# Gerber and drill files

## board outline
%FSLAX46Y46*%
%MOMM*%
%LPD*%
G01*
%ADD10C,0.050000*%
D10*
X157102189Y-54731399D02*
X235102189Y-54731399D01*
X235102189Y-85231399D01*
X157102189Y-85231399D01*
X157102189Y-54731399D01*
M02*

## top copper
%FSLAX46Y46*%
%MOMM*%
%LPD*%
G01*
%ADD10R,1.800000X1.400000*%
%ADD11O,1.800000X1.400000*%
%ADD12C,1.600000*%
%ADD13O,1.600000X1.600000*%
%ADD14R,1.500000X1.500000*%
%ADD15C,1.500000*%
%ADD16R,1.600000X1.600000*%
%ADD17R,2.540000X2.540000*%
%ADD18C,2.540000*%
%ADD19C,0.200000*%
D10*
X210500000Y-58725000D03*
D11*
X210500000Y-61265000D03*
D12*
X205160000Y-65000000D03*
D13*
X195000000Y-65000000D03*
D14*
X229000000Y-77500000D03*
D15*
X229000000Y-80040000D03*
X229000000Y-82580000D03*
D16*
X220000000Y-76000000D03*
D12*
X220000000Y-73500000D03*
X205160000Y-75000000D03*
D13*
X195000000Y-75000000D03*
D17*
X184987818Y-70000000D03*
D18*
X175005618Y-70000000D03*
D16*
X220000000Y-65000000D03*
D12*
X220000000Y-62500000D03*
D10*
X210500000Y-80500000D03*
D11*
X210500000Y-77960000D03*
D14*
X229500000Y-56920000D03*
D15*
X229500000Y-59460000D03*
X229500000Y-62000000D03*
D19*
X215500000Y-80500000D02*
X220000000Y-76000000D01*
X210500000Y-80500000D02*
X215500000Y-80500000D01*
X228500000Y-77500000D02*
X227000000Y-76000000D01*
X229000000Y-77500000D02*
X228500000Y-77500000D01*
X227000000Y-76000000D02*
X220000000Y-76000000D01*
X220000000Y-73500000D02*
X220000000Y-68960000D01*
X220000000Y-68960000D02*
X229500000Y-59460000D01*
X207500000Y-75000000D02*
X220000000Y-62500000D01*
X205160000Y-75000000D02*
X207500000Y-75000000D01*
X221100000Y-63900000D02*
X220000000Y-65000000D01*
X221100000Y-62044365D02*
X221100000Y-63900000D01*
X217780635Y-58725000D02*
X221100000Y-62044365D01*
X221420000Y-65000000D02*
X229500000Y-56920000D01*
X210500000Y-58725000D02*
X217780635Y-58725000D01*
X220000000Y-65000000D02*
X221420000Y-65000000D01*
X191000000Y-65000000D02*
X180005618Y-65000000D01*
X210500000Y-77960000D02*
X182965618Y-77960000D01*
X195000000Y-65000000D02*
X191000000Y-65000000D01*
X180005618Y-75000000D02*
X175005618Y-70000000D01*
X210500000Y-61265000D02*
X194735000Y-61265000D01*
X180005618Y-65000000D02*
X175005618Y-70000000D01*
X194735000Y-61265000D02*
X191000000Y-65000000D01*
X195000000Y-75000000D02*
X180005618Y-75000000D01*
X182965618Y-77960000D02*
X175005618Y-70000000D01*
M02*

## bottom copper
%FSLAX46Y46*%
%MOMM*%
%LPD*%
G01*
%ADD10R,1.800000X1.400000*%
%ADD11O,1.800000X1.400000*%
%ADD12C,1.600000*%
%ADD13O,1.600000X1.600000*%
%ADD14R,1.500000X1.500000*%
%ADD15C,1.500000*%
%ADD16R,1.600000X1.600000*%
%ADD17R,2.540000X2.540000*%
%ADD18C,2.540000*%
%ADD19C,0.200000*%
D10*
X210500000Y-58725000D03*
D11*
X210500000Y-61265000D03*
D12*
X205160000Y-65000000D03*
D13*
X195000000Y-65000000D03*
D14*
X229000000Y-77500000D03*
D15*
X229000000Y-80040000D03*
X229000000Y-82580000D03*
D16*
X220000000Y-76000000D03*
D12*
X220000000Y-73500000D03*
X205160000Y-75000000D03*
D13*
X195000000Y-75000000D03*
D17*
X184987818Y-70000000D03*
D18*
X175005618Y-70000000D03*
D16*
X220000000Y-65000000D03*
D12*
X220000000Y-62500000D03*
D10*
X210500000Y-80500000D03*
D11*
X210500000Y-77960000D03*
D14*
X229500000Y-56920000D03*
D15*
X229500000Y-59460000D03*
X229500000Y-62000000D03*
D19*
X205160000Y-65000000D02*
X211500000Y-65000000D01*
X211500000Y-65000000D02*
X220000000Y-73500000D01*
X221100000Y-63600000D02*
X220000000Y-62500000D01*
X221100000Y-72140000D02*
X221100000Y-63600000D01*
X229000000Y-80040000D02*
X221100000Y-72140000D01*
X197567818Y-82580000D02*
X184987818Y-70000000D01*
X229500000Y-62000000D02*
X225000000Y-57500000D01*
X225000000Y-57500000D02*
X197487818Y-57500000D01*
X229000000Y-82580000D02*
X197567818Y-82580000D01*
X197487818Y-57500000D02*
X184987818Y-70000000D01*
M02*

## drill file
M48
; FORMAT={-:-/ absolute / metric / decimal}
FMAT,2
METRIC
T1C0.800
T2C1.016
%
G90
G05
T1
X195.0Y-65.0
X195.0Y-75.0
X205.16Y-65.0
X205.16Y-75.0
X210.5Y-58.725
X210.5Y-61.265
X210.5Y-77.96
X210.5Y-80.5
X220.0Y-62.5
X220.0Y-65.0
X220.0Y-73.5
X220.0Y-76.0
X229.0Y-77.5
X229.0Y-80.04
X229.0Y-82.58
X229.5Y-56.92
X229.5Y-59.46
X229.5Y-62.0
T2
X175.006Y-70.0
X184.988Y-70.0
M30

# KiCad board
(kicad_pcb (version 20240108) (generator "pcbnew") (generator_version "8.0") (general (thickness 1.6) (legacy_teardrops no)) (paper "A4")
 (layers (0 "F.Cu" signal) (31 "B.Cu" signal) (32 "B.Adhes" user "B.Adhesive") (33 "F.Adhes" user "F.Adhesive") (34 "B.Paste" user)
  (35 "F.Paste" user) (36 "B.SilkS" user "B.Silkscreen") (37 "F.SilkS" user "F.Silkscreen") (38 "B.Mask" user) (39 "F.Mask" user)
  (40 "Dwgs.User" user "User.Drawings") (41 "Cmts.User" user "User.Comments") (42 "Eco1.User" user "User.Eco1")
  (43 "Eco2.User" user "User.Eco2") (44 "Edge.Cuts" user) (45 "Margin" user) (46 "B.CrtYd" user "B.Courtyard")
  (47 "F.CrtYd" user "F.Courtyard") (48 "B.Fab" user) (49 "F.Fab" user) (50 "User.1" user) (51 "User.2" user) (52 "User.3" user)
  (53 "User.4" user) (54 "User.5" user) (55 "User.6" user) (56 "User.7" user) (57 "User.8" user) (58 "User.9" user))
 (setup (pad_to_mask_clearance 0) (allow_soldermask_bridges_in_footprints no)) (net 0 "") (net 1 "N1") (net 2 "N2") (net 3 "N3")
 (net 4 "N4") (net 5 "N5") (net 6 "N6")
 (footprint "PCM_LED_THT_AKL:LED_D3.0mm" (layer "F.Cu") (at 210.5 58.725 -90)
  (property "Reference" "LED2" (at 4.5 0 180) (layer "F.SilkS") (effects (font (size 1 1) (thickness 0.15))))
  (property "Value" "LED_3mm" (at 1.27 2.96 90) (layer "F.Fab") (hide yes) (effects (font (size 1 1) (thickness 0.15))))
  (pad "1" thru_hole rect (at 0 0 270) (size 1.4 1.8) (drill 0.8) (layers "*.Cu" "*.Mask") (remove_unused_layers no) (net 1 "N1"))
  (pad "2" thru_hole oval (at 2.54 0 270) (size 1.4 1.8) (drill 0.8) (layers "*.Cu" "*.Mask") (remove_unused_layers no) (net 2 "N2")))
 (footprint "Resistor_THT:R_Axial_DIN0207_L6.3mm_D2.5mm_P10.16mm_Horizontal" (layer "F.Cu") (at 205.16 65 180)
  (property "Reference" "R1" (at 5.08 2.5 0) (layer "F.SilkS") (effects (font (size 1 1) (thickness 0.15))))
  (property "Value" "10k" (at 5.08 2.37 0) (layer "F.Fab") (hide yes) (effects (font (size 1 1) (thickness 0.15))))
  (pad "1" thru_hole circle (at 0 0 180) (size 1.6 1.6) (drill 0.8) (layers "*.Cu" "*.Mask") (remove_unused_layers no) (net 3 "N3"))
  (pad "2" thru_hole oval (at 10.16 0 180) (size 1.6 1.6) (drill 0.8) (layers "*.Cu" "*.Mask") (remove_unused_layers no) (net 2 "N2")))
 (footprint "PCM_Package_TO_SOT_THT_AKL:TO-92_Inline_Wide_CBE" (layer "F.Cu") (at 229 77.5 -90)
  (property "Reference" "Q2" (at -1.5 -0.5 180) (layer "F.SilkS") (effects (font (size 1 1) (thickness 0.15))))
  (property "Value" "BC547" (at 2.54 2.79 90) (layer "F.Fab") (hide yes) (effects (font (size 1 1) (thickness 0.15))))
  (pad "1" thru_hole rect (at 0 0) (size 1.5 1.5) (drill 0.8) (layers "*.Cu" "*.Mask") (remove_unused_layers no) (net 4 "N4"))
  (pad "2" thru_hole circle (at 2.54 0) (size 1.5 1.5) (drill 0.8) (layers "*.Cu" "*.Mask") (remove_unused_layers no) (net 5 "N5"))
  (pad "3" thru_hole circle (at 5.08 0) (size 1.5 1.5) (drill 0.8) (layers "*.Cu" "*.Mask") (remove_unused_layers no) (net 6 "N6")))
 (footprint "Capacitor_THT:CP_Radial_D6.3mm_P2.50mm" (layer "F.Cu") (at 220 76 90)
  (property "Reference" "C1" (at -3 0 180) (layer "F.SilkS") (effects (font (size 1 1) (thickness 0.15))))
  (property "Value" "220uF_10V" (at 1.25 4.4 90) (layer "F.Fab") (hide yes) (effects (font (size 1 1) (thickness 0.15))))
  (pad "1" thru_hole rect (at 0 0 90) (size 1.6 1.6) (drill 0.8) (layers "*.Cu" "*.Mask") (remove_unused_layers no) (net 4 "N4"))
  (pad "2" thru_hole circle (at 2.5 0 90) (size 1.6 1.6) (drill 0.8) (layers "*.Cu" "*.Mask") (remove_unused_layers no) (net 3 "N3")))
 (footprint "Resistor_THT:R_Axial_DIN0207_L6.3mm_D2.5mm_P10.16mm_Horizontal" (layer "F.Cu") (at 205.16 75 180)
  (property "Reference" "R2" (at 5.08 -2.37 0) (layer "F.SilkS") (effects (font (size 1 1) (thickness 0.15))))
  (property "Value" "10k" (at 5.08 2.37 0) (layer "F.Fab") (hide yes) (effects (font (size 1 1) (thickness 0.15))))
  (pad "1" thru_hole circle (at 0 0 180) (size 1.6 1.6) (drill 0.8) (layers "*.Cu" "*.Mask") (remove_unused_layers no) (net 5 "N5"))
  (pad "2" thru_hole oval (at 10.16 0 180) (size 1.6 1.6) (drill 0.8) (layers "*.Cu" "*.Mask") (remove_unused_layers no) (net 2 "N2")))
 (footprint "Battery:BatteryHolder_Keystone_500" (layer "F.Cu") (at 184.987818 70 180)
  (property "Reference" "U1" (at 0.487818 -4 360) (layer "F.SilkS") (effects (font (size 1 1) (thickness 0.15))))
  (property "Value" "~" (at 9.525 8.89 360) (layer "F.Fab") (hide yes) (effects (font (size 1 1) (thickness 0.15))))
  (pad "1" thru_hole rect (at 0 0 180) (size 2.54 2.54) (drill 1.016) (layers "*.Cu" "*.Mask") (remove_unused_layers no) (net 6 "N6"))
  (pad "2" thru_hole circle (at 9.9822 0 180) (size 2.54 2.54) (drill 1.016) (layers "*.Cu" "*.Mask") (remove_unused_layers no) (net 2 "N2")))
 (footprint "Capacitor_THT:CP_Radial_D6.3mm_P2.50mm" (layer "F.Cu") (at 220 65 90)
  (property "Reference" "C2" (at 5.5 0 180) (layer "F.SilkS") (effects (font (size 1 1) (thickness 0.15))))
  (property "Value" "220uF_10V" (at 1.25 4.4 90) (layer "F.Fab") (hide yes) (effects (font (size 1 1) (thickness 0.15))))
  (pad "1" thru_hole rect (at 0 0 90) (size 1.6 1.6) (drill 0.8) (layers "*.Cu" "*.Mask") (remove_unused_layers no) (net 1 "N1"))
  (pad "2" thru_hole circle (at 2.5 0 90) (size 1.6 1.6) (drill 0.8) (layers "*.Cu" "*.Mask") (remove_unused_layers no) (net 5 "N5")))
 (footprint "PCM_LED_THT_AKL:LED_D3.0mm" (layer "F.Cu") (at 210.5 80.5 90)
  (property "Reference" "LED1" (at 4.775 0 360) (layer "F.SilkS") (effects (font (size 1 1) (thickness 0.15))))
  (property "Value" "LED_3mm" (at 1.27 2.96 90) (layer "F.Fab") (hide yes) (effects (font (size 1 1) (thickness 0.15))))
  (pad "1" thru_hole rect (at 0 0 90) (size 1.4 1.8) (drill 0.8) (layers "*.Cu" "*.Mask") (remove_unused_layers no) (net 4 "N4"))
  (pad "2" thru_hole oval (at 2.54 0 90) (size 1.4 1.8) (drill 0.8) (layers "*.Cu" "*.Mask") (remove_unused_layers no) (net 2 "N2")))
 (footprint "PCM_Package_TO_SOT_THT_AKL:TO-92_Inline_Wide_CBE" (layer "F.Cu") (at 229.5 56.92 -90)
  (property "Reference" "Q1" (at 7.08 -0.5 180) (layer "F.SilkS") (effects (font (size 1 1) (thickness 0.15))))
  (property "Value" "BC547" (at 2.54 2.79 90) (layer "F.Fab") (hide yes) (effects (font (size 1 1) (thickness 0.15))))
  (pad "1" thru_hole rect (at 0 0) (size 1.5 1.5) (drill 0.8) (layers "*.Cu" "*.Mask") (remove_unused_layers no) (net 1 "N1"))
  (pad "2" thru_hole circle (at 2.54 0) (size 1.5 1.5) (drill 0.8) (layers "*.Cu" "*.Mask") (remove_unused_layers no) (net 3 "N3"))
  (pad "3" thru_hole circle (at 5.08 0) (size 1.5 1.5) (drill 0.8) (layers "*.Cu" "*.Mask") (remove_unused_layers no) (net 6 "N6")))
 (gr_rect (start 157.102189 54.731399) (end 235.102189 85.231399) (stroke (width 0.05) (type default)) (fill none) (layer "Edge.Cuts"))
 (segment (start 215.5 80.5) (end 220 76) (width 0.2) (layer "F.Cu") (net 4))
 (segment (start 210.5 80.5) (end 215.5 80.5) (width 0.2) (layer "F.Cu") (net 4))
 (segment (start 228.5 77.5) (end 227 76) (width 0.2) (layer "F.Cu") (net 4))
 (segment (start 229 77.5) (end 228.5 77.5) (width 0.2) (layer "F.Cu") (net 4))
 (segment (start 227 76) (end 220 76) (width 0.2) (layer "F.Cu") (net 4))
 (segment (start 220 73.5) (end 220 68.96) (width 0.2) (layer "F.Cu") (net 3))
 (segment (start 220 68.96) (end 229.5 59.46) (width 0.2) (layer "F.Cu") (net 3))
 (segment (start 205.16 65) (end 211.5 65) (width 0.2) (layer "B.Cu") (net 3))
 (segment (start 211.5 65) (end 220 73.5) (width 0.2) (layer "B.Cu") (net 3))
 (segment (start 207.5 75) (end 220 62.5) (width 0.2) (layer "F.Cu") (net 5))
 (segment (start 205.16 75) (end 207.5 75) (width 0.2) (layer "F.Cu") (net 5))
 (segment (start 221.1 63.6) (end 220 62.5) (width 0.2) (layer "B.Cu") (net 5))
 (segment (start 221.1 72.14) (end 221.1 63.6) (width 0.2) (layer "B.Cu") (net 5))
 (segment (start 229 80.04) (end 221.1 72.14) (width 0.2) (layer "B.Cu") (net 5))
 (segment (start 221.1 63.9) (end 220 65) (width 0.2) (layer "F.Cu") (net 1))
 (segment (start 221.1 62.044365) (end 221.1 63.9) (width 0.2) (layer "F.Cu") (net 1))
 (segment (start 217.780635 58.725) (end 221.1 62.044365) (width 0.2) (layer "F.Cu") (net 1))
 (segment (start 221.42 65) (end 229.5 56.92) (width 0.2) (layer "F.Cu") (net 1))
 (segment (start 210.5 58.725) (end 217.780635 58.725) (width 0.2) (layer "F.Cu") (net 1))
 (segment (start 220 65) (end 221.42 65) (width 0.2) (layer "F.Cu") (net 1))
 (segment (start 191 65) (end 180.005618 65) (width 0.2) (layer "F.Cu") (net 2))
 (segment (start 210.5 77.96) (end 182.965618 77.96) (width 0.2) (layer "F.Cu") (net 2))
 (segment (start 195 65) (end 191 65) (width 0.2) (layer "F.Cu") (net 2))
 (segment (start 180.005618 75) (end 175.005618 70) (width 0.2) (layer "F.Cu") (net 2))
 (segment (start 210.5 61.265) (end 194.735 61.265) (width 0.2) (layer "F.Cu") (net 2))
 (segment (start 180.005618 65) (end 175.005618 70) (width 0.2) (layer "F.Cu") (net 2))
 (segment (start 194.735 61.265) (end 191 65) (width 0.2) (layer "F.Cu") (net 2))
 (segment (start 195 75) (end 180.005618 75) (width 0.2) (layer "F.Cu") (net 2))
 (segment (start 182.965618 77.96) (end 175.005618 70) (width 0.2) (layer "F.Cu") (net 2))
 (segment (start 197.567818 82.58) (end 184.987818 70) (width 0.2) (layer "B.Cu") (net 6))
 (segment (start 229.5 62) (end 225 57.5) (width 0.2) (layer "B.Cu") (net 6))
 (segment (start 225 57.5) (end 197.487818 57.5) (width 0.2) (layer "B.Cu") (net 6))
 (segment (start 229 82.58) (end 197.567818 82.58) (width 0.2) (layer "B.Cu") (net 6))
 (segment (start 197.487818 57.5) (end 184.987818 70) (width 0.2) (layer "B.Cu") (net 6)))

